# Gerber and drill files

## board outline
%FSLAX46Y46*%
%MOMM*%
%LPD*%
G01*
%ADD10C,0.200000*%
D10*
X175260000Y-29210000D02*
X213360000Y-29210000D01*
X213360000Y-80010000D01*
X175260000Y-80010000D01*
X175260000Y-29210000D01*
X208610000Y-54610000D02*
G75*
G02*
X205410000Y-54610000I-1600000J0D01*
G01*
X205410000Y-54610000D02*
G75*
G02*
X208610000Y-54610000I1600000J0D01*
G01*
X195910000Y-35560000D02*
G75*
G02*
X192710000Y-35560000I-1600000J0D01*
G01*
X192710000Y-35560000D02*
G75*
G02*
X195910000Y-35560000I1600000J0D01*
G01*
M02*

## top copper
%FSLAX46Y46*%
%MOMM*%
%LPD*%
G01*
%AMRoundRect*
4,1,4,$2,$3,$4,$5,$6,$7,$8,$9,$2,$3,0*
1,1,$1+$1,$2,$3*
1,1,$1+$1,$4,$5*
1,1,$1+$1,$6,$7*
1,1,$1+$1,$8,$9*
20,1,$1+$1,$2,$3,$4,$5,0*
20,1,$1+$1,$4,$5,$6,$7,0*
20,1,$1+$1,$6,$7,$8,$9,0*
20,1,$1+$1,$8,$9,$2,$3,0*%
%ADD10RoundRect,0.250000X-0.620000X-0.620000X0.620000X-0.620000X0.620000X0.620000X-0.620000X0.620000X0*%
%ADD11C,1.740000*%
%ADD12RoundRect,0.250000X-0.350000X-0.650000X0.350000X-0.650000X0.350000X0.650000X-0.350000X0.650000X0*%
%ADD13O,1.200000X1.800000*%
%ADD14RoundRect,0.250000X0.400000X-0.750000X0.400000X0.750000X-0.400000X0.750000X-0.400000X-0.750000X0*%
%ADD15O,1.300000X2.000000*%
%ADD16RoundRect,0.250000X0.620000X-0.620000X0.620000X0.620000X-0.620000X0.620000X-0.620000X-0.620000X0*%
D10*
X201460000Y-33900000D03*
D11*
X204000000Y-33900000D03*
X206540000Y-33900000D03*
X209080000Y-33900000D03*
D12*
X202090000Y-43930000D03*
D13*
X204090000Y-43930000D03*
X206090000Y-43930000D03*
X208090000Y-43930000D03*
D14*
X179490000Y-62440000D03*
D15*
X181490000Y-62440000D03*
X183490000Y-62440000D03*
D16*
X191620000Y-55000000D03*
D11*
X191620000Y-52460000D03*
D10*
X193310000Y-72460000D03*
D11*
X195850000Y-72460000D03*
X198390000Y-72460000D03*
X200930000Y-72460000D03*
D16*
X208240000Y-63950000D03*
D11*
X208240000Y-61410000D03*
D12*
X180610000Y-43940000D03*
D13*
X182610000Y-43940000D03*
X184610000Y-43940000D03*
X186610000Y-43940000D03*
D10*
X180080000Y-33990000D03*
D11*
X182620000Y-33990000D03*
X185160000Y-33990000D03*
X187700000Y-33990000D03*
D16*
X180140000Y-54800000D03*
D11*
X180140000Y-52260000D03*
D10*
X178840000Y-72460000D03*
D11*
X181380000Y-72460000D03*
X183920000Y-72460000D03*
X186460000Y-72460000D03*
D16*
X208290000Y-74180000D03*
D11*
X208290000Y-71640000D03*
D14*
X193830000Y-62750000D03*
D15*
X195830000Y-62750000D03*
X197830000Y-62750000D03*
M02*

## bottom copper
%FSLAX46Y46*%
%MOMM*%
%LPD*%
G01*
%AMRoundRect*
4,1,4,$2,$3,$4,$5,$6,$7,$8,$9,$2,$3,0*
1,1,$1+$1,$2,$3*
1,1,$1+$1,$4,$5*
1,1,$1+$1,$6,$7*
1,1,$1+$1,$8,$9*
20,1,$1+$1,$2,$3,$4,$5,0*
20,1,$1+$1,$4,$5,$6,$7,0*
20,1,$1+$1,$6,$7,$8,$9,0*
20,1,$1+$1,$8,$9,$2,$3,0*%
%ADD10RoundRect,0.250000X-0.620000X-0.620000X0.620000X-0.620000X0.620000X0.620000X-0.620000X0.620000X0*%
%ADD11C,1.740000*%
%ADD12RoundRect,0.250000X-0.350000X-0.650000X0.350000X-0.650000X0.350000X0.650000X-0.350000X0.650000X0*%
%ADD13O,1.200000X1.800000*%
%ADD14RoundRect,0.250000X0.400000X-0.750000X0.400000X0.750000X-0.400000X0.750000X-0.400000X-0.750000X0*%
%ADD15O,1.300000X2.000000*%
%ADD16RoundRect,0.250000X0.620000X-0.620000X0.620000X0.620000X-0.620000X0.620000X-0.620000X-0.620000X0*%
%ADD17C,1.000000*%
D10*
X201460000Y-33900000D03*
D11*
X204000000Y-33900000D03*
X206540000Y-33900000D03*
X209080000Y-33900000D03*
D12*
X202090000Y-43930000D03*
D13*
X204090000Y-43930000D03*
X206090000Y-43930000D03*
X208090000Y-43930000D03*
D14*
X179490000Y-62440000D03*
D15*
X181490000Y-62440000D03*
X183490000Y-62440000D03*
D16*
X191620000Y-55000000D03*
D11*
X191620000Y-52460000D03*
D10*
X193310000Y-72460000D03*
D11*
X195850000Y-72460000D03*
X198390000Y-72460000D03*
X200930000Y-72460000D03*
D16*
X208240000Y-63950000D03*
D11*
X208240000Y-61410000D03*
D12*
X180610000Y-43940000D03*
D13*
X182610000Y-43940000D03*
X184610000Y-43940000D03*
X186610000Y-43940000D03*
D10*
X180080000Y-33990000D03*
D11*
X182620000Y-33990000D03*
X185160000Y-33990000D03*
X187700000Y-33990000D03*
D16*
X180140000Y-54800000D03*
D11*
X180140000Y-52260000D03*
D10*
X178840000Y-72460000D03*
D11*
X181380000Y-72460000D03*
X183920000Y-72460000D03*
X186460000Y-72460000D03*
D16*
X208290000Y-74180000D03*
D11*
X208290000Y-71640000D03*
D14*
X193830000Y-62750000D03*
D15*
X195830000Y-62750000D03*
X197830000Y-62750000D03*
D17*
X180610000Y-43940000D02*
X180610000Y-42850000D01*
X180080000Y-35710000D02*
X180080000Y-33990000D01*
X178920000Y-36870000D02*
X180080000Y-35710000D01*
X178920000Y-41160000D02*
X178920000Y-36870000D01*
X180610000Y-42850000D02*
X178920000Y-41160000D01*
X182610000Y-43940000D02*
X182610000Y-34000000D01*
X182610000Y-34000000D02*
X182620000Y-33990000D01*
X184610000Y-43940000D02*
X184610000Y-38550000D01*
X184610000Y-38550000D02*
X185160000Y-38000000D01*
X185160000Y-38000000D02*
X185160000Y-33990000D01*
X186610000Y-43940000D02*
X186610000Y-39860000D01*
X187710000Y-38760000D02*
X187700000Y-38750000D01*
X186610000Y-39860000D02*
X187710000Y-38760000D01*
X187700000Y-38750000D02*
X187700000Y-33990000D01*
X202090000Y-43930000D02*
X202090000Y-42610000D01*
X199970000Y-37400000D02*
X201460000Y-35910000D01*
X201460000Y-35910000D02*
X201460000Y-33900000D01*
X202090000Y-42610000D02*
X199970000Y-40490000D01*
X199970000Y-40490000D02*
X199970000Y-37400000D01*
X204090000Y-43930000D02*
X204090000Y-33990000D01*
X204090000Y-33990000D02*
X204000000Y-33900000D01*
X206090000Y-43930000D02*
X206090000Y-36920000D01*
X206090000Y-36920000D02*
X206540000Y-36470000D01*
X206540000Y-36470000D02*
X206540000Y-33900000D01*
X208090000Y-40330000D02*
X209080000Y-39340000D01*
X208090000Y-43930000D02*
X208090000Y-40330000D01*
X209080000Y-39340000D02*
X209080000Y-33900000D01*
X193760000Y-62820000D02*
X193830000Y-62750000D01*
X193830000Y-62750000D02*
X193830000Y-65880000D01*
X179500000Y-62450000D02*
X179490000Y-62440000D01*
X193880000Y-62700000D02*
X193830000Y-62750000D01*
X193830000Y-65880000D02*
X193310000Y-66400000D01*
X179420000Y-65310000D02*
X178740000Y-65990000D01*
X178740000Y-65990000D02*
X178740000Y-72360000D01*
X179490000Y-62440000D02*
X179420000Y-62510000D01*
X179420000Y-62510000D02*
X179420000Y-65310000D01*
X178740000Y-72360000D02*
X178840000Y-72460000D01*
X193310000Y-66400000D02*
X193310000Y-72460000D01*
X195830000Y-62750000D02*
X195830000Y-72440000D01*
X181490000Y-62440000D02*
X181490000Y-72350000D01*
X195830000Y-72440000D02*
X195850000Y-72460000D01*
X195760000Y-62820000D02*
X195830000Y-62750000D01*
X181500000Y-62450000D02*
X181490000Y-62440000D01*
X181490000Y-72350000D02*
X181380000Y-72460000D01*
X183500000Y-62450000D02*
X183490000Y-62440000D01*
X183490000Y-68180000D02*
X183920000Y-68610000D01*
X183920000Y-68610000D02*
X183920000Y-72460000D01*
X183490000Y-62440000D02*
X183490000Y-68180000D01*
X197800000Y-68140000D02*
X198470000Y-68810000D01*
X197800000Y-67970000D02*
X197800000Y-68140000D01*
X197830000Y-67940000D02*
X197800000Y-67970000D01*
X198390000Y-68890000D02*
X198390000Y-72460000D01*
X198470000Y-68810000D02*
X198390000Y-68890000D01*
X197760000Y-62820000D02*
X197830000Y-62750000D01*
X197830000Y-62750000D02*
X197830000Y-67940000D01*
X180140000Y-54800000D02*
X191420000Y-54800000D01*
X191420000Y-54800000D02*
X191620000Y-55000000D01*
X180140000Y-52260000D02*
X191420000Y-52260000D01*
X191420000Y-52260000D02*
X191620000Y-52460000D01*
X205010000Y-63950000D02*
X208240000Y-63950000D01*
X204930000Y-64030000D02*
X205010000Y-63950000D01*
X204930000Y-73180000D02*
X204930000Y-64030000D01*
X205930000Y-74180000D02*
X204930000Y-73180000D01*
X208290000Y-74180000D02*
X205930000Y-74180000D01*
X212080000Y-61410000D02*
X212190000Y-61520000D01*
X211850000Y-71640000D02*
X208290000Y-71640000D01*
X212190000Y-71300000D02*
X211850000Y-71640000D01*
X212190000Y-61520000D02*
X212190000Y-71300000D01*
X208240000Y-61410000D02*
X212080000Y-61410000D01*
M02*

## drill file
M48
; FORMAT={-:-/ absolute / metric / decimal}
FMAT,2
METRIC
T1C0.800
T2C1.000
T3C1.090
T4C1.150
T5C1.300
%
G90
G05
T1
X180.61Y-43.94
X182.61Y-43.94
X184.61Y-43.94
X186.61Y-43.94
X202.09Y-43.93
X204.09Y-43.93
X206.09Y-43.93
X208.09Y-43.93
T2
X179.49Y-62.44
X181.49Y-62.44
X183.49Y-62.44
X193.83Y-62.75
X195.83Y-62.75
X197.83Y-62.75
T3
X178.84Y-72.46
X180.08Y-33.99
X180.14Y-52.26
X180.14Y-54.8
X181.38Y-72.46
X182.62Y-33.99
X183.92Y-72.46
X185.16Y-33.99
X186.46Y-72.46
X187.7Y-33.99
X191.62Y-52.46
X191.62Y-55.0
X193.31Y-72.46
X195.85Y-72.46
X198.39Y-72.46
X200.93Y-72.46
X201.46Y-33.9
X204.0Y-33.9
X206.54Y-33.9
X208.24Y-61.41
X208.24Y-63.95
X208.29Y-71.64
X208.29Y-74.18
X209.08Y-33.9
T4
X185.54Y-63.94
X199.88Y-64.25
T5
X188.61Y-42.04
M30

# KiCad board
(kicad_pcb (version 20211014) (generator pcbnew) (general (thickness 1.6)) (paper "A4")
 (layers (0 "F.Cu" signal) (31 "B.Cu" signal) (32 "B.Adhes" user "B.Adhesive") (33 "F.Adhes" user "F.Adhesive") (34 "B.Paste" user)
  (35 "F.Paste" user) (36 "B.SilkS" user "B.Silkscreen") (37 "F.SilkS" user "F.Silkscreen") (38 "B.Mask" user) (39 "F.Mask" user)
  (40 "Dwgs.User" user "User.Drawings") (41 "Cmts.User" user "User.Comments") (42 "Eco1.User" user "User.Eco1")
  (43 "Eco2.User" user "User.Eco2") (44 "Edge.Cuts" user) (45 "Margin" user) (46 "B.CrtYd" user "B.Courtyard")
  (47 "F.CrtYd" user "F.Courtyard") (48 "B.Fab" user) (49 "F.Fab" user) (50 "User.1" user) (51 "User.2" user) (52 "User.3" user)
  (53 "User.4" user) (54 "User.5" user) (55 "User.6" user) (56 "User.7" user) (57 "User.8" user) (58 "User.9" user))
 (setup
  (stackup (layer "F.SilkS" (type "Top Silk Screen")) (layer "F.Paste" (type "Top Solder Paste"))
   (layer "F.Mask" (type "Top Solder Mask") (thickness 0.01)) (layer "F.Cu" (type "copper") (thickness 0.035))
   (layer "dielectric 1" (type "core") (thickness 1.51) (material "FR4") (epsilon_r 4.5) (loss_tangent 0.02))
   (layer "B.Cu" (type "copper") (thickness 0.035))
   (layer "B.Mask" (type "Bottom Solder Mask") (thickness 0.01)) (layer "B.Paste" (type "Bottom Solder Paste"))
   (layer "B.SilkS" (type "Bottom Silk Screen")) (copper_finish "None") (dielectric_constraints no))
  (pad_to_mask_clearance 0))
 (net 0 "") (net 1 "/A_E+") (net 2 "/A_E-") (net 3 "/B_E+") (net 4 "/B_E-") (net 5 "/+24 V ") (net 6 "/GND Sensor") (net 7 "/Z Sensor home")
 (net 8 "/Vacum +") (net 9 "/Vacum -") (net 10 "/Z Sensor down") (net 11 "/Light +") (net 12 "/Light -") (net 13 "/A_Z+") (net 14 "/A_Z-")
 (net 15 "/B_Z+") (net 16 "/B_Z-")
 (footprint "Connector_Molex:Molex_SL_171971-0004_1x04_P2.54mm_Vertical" (layer "F.Cu") (at 201.46 33.9)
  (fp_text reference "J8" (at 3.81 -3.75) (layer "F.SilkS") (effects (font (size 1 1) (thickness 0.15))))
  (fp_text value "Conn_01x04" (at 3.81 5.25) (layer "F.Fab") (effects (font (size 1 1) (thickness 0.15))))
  (pad "1" thru_hole roundrect (at 0 0) (size 1.74 1.74) (drill 1.09) (layers *.Cu *.Mask) (roundrect_rratio 0.1436781609) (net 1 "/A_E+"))
  (pad "2" thru_hole circle (at 2.54 0) (size 1.74 1.74) (drill 1.09) (layers *.Cu *.Mask) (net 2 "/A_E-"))
  (pad "3" thru_hole circle (at 5.08 0) (size 1.74 1.74) (drill 1.09) (layers *.Cu *.Mask) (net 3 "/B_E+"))
  (pad "4" thru_hole circle (at 7.62 0) (size 1.74 1.74) (drill 1.09) (layers *.Cu *.Mask) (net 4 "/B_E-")))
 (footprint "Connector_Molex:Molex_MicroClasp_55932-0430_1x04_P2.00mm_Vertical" (layer "F.Cu") (at 202.09 43.93)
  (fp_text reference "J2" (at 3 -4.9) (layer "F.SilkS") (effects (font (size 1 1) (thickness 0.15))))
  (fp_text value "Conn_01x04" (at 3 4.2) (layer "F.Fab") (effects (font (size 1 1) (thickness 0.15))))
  (pad "1" thru_hole roundrect (at 0 0) (size 1.2 1.8) (drill 0.8) (layers *.Cu *.Mask) (roundrect_rratio 0.2083333333) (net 1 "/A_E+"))
  (pad "2" thru_hole oval (at 2 0) (size 1.2 1.8) (drill 0.8) (layers *.Cu *.Mask) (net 2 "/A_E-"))
  (pad "3" thru_hole oval (at 4 0) (size 1.2 1.8) (drill 0.8) (layers *.Cu *.Mask) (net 3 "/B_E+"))
  (pad "4" thru_hole oval (at 6 0) (size 1.2 1.8) (drill 0.8) (layers *.Cu *.Mask) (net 4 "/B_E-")))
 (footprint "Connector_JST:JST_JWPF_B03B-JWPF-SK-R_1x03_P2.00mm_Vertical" (layer "F.Cu") (at 179.49 62.44 90)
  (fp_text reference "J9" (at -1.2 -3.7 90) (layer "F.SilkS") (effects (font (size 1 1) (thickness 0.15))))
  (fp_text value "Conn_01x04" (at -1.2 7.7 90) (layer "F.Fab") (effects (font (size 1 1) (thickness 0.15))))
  (pad "" np_thru_hole circle (at -1.5 6.05 90) (size 1.15 1.15) (drill 1.15) (layers *.Cu *.Mask))
  (pad "1" thru_hole roundrect (at 0 0 90) (size 2 1.3) (drill 1) (layers *.Cu *.Mask) (roundrect_rratio 0.1923076923) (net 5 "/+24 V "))
  (pad "2" thru_hole oval (at 0 2 90) (size 2 1.3) (drill 1) (layers *.Cu *.Mask) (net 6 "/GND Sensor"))
  (pad "3" thru_hole oval (at 0 4 90) (size 2 1.3) (drill 1) (layers *.Cu *.Mask) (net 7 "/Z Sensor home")))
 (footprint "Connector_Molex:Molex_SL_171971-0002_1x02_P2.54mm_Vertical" (layer "F.Cu") (at 191.62 55 90)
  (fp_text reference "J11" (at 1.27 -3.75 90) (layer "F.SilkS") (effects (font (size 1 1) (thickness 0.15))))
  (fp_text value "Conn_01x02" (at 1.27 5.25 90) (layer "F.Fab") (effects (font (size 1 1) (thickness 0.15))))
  (pad "1" thru_hole roundrect (at 0 0 90) (size 1.74 1.74) (drill 1.09) (layers *.Cu *.Mask) (roundrect_rratio 0.1436781609)
   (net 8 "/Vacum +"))
  (pad "2" thru_hole circle (at 2.54 0 90) (size 1.74 1.74) (drill 1.09) (layers *.Cu *.Mask) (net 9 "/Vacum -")))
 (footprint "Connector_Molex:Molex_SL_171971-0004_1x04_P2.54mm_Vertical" (layer "F.Cu") (at 193.31 72.46)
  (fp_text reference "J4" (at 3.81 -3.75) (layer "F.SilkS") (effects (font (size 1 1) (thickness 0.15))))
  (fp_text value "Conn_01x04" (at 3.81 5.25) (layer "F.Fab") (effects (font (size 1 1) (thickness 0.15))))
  (pad "1" thru_hole roundrect (at 0 0) (size 1.74 1.74) (drill 1.09) (layers *.Cu *.Mask) (roundrect_rratio 0.1436781609) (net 5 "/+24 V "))
  (pad "2" thru_hole circle (at 2.54 0) (size 1.74 1.74) (drill 1.09) (layers *.Cu *.Mask) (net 6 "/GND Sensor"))
  (pad "3" thru_hole circle (at 5.08 0) (size 1.74 1.74) (drill 1.09) (layers *.Cu *.Mask) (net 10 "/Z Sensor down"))
  (pad "4" thru_hole circle (at 7.62 0) (size 1.74 1.74) (drill 1.09) (layers *.Cu *.Mask)))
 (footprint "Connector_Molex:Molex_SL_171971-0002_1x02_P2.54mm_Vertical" (layer "F.Cu") (at 208.24 63.95 90)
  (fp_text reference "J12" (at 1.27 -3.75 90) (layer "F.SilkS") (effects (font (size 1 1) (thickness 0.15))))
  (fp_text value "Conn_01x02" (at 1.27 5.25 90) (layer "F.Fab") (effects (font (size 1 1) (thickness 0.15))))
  (pad "1" thru_hole roundrect (at 0 0 90) (size 1.74 1.74) (drill 1.09) (layers *.Cu *.Mask) (roundrect_rratio 0.1436781609)
   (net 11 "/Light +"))
  (pad "2" thru_hole circle (at 2.54 0 90) (size 1.74 1.74) (drill 1.09) (layers *.Cu *.Mask) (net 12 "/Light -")))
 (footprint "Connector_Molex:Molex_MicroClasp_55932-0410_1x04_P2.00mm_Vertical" (layer "F.Cu") (at 180.61 43.94)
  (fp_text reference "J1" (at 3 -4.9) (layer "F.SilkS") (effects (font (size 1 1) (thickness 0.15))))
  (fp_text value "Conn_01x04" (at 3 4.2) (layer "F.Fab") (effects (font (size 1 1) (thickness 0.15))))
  (pad "" np_thru_hole circle (at 8 -1.9) (size 1.3 1.3) (drill 1.3) (layers *.Cu *.Mask))
  (pad "1" thru_hole roundrect (at 0 0) (size 1.2 1.8) (drill 0.8) (layers *.Cu *.Mask) (roundrect_rratio 0.2083333333) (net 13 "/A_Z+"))
  (pad "2" thru_hole oval (at 2 0) (size 1.2 1.8) (drill 0.8) (layers *.Cu *.Mask) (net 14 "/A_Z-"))
  (pad "3" thru_hole oval (at 4 0) (size 1.2 1.8) (drill 0.8) (layers *.Cu *.Mask) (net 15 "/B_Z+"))
  (pad "4" thru_hole oval (at 6 0) (size 1.2 1.8) (drill 0.8) (layers *.Cu *.Mask) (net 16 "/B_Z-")))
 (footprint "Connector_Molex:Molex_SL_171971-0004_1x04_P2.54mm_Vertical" (layer "F.Cu") (at 180.08 33.99)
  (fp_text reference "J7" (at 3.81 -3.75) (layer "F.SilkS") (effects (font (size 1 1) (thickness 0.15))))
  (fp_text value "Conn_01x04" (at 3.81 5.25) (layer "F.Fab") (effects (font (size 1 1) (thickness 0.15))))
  (pad "1" thru_hole roundrect (at 0 0) (size 1.74 1.74) (drill 1.09) (layers *.Cu *.Mask) (roundrect_rratio 0.1436781609) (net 13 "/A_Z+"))
  (pad "2" thru_hole circle (at 2.54 0) (size 1.74 1.74) (drill 1.09) (layers *.Cu *.Mask) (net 14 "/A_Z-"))
  (pad "3" thru_hole circle (at 5.08 0) (size 1.74 1.74) (drill 1.09) (layers *.Cu *.Mask) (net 15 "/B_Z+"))
  (pad "4" thru_hole circle (at 7.62 0) (size 1.74 1.74) (drill 1.09) (layers *.Cu *.Mask) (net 16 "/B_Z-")))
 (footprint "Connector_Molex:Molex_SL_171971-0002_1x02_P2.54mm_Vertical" (layer "F.Cu") (at 180.14 54.8 90)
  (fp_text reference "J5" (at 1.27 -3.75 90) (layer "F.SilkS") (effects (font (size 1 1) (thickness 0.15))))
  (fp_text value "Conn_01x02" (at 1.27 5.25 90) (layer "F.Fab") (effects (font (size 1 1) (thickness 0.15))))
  (pad "1" thru_hole roundrect (at 0 0 90) (size 1.74 1.74) (drill 1.09) (layers *.Cu *.Mask) (roundrect_rratio 0.1436781609)
   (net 8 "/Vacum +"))
  (pad "2" thru_hole circle (at 2.54 0 90) (size 1.74 1.74) (drill 1.09) (layers *.Cu *.Mask) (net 9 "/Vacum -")))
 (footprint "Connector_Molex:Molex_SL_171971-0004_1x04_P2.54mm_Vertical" (layer "F.Cu") (at 178.84 72.46)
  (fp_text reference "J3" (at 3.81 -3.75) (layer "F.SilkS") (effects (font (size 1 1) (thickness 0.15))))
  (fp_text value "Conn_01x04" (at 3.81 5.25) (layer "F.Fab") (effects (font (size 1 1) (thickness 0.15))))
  (pad "1" thru_hole roundrect (at 0 0) (size 1.74 1.74) (drill 1.09) (layers *.Cu *.Mask) (roundrect_rratio 0.1436781609) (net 5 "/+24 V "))
  (pad "2" thru_hole circle (at 2.54 0) (size 1.74 1.74) (drill 1.09) (layers *.Cu *.Mask) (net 6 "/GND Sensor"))
  (pad "3" thru_hole circle (at 5.08 0) (size 1.74 1.74) (drill 1.09) (layers *.Cu *.Mask) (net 7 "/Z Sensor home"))
  (pad "4" thru_hole circle (at 7.62 0) (size 1.74 1.74) (drill 1.09) (layers *.Cu *.Mask)))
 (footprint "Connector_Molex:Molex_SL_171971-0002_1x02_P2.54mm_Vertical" (layer "F.Cu") (at 208.29 74.18 90)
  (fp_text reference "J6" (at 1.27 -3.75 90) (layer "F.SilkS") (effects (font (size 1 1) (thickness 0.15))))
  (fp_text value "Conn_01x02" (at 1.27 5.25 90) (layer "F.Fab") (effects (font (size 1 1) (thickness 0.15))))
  (pad "1" thru_hole roundrect (at 0 0 90) (size 1.74 1.74) (drill 1.09) (layers *.Cu *.Mask) (roundrect_rratio 0.1436781609)
   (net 11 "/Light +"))
  (pad "2" thru_hole circle (at 2.54 0 90) (size 1.74 1.74) (drill 1.09) (layers *.Cu *.Mask) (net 12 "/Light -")))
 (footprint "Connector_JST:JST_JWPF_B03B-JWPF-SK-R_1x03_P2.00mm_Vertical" (layer "F.Cu") (at 193.83 62.75 90)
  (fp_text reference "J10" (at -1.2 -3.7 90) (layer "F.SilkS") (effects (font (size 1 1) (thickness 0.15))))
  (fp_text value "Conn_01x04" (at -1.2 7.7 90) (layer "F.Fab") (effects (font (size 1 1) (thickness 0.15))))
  (pad "" np_thru_hole circle (at -1.5 6.05 90) (size 1.15 1.15) (drill 1.15) (layers *.Cu *.Mask))
  (pad "1" thru_hole roundrect (at 0 0 90) (size 2 1.3) (drill 1) (layers *.Cu *.Mask) (roundrect_rratio 0.1923076923) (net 5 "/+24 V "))
  (pad "2" thru_hole oval (at 0 2 90) (size 2 1.3) (drill 1) (layers *.Cu *.Mask) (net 6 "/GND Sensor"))
  (pad "3" thru_hole oval (at 0 4 90) (size 2 1.3) (drill 1) (layers *.Cu *.Mask) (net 10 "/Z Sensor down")))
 (gr_rect (start 175.26 29.21) (end 213.36 80.01) (layer "Edge.Cuts") (width 0.2) (fill none))
 (gr_circle (center 207.01 54.61) (end 208.61 54.61) (layer "Edge.Cuts") (width 0.2) (fill none))
 (gr_circle (center 194.31 35.56) (end 195.91 35.56) (layer "Edge.Cuts") (width 0.2) (fill none))
 (segment (start 180.61 43.94) (end 180.61 42.85) (width 1) (layer "B.Cu") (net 13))
 (segment (start 180.08 35.71) (end 180.08 33.99) (width 1) (layer "B.Cu") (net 13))
 (segment (start 178.92 36.87) (end 180.08 35.71) (width 1) (layer "B.Cu") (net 13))
 (segment (start 178.92 41.16) (end 178.92 36.87) (width 1) (layer "B.Cu") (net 13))
 (segment (start 180.61 42.85) (end 178.92 41.16) (width 1) (layer "B.Cu") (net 13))
 (segment (start 182.61 43.94) (end 182.61 34) (width 1) (layer "B.Cu") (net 14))
 (segment (start 182.61 34) (end 182.62 33.99) (width 1) (layer "B.Cu") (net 14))
 (segment (start 184.61 43.94) (end 184.61 38.55) (width 1) (layer "B.Cu") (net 15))
 (segment (start 184.61 38.55) (end 185.16 38) (width 1) (layer "B.Cu") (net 15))
 (segment (start 185.16 38) (end 185.16 33.99) (width 1) (layer "B.Cu") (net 15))
 (segment (start 186.61 43.94) (end 186.61 39.86) (width 1) (layer "B.Cu") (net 16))
 (segment (start 187.71 38.76) (end 187.7 38.75) (width 1) (layer "B.Cu") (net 16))
 (segment (start 186.61 39.86) (end 187.71 38.76) (width 1) (layer "B.Cu") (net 16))
 (segment (start 187.7 38.75) (end 187.7 33.99) (width 1) (layer "B.Cu") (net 16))
 (segment (start 202.09 43.93) (end 202.09 42.61) (width 1) (layer "B.Cu") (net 1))
 (segment (start 199.97 37.4) (end 201.46 35.91) (width 1) (layer "B.Cu") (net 1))
 (segment (start 201.46 35.91) (end 201.46 33.9) (width 1) (layer "B.Cu") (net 1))
 (segment (start 202.09 42.61) (end 199.97 40.49) (width 1) (layer "B.Cu") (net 1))
 (segment (start 199.97 40.49) (end 199.97 37.4) (width 1) (layer "B.Cu") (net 1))
 (segment (start 204.09 43.93) (end 204.09 33.99) (width 1) (layer "B.Cu") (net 2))
 (segment (start 204.09 33.99) (end 204 33.9) (width 1) (layer "B.Cu") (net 2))
 (segment (start 206.09 43.93) (end 206.09 36.92) (width 1) (layer "B.Cu") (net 3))
 (segment (start 206.09 36.92) (end 206.54 36.47) (width 1) (layer "B.Cu") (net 3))
 (segment (start 206.54 36.47) (end 206.54 33.9) (width 1) (layer "B.Cu") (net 3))
 (segment (start 208.09 40.33) (end 209.08 39.34) (width 1) (layer "B.Cu") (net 4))
 (segment (start 208.09 43.93) (end 208.09 40.33) (width 1) (layer "B.Cu") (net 4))
 (segment (start 209.08 39.34) (end 209.08 33.9) (width 1) (layer "B.Cu") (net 4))
 (segment (start 193.76 62.82) (end 193.83 62.75) (width 1) (layer "B.Cu") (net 5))
 (segment (start 193.83 62.75) (end 193.83 65.88) (width 1) (layer "B.Cu") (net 5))
 (segment (start 179.5 62.45) (end 179.49 62.44) (width 1) (layer "B.Cu") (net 5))
 (segment (start 193.88 62.7) (end 193.83 62.75) (width 1) (layer "B.Cu") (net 5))
 (segment (start 193.83 65.88) (end 193.31 66.4) (width 1) (layer "B.Cu") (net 5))
 (segment (start 179.42 65.31) (end 178.74 65.99) (width 1) (layer "B.Cu") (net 5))
 (segment (start 178.74 65.99) (end 178.74 72.36) (width 1) (layer "B.Cu") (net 5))
 (segment (start 179.49 62.44) (end 179.42 62.51) (width 1) (layer "B.Cu") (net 5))
 (segment (start 179.42 62.51) (end 179.42 65.31) (width 1) (layer "B.Cu") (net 5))
 (segment (start 178.74 72.36) (end 178.84 72.46) (width 1) (layer "B.Cu") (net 5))
 (segment (start 193.31 66.4) (end 193.31 72.46) (width 1) (layer "B.Cu") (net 5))
 (segment (start 195.83 62.75) (end 195.83 72.44) (width 1) (layer "B.Cu") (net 6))
 (segment (start 181.49 62.44) (end 181.49 72.35) (width 1) (layer "B.Cu") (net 6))
 (segment (start 195.83 72.44) (end 195.85 72.46) (width 1) (layer "B.Cu") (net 6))
 (segment (start 195.76 62.82) (end 195.83 62.75) (width 1) (layer "B.Cu") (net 6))
 (segment (start 181.5 62.45) (end 181.49 62.44) (width 1) (layer "B.Cu") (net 6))
 (segment (start 181.49 72.35) (end 181.38 72.46) (width 1) (layer "B.Cu") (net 6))
 (segment (start 183.5 62.45) (end 183.49 62.44) (width 1) (layer "B.Cu") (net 7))
 (segment (start 183.49 68.18) (end 183.92 68.61) (width 1) (layer "B.Cu") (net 7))
 (segment (start 183.92 68.61) (end 183.92 72.46) (width 1) (layer "B.Cu") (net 7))
 (segment (start 183.49 62.44) (end 183.49 68.18) (width 1) (layer "B.Cu") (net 7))
 (segment (start 197.8 68.14) (end 198.47 68.81) (width 1) (layer "B.Cu") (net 10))
 (segment (start 197.8 67.97) (end 197.8 68.14) (width 1) (layer "B.Cu") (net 10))
 (segment (start 197.83 67.94) (end 197.8 67.97) (width 1) (layer "B.Cu") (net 10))
 (segment (start 198.39 68.89) (end 198.39 72.46) (width 1) (layer "B.Cu") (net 10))
 (segment (start 198.47 68.81) (end 198.39 68.89) (width 1) (layer "B.Cu") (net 10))
 (segment (start 197.76 62.82) (end 197.83 62.75) (width 1) (layer "B.Cu") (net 10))
 (segment (start 197.83 62.75) (end 197.83 67.94) (width 1) (layer "B.Cu") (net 10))
 (segment (start 180.14 54.8) (end 191.42 54.8) (width 1) (layer "B.Cu") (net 8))
 (segment (start 191.42 54.8) (end 191.62 55) (width 1) (layer "B.Cu") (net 8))
 (segment (start 180.14 52.26) (end 191.42 52.26) (width 1) (layer "B.Cu") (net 9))
 (segment (start 191.42 52.26) (end 191.62 52.46) (width 1) (layer "B.Cu") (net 9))
 (segment (start 205.01 63.95) (end 208.24 63.95) (width 1) (layer "B.Cu") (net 11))
 (segment (start 204.93 64.03) (end 205.01 63.95) (width 1) (layer "B.Cu") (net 11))
 (segment (start 204.93 73.18) (end 204.93 64.03) (width 1) (layer "B.Cu") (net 11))
 (segment (start 205.93 74.18) (end 204.93 73.18) (width 1) (layer "B.Cu") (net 11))
 (segment (start 208.29 74.18) (end 205.93 74.18) (width 1) (layer "B.Cu") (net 11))
 (segment (start 212.08 61.41) (end 212.19 61.52) (width 1) (layer "B.Cu") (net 12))
 (segment (start 211.85 71.64) (end 208.29 71.64) (width 1) (layer "B.Cu") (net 12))
 (segment (start 212.19 71.3) (end 211.85 71.64) (width 1) (layer "B.Cu") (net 12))
 (segment (start 212.19 61.52) (end 212.19 71.3) (width 1) (layer "B.Cu") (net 12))
 (segment (start 208.24 61.41) (end 212.08 61.41) (width 1) (layer "B.Cu") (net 12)))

